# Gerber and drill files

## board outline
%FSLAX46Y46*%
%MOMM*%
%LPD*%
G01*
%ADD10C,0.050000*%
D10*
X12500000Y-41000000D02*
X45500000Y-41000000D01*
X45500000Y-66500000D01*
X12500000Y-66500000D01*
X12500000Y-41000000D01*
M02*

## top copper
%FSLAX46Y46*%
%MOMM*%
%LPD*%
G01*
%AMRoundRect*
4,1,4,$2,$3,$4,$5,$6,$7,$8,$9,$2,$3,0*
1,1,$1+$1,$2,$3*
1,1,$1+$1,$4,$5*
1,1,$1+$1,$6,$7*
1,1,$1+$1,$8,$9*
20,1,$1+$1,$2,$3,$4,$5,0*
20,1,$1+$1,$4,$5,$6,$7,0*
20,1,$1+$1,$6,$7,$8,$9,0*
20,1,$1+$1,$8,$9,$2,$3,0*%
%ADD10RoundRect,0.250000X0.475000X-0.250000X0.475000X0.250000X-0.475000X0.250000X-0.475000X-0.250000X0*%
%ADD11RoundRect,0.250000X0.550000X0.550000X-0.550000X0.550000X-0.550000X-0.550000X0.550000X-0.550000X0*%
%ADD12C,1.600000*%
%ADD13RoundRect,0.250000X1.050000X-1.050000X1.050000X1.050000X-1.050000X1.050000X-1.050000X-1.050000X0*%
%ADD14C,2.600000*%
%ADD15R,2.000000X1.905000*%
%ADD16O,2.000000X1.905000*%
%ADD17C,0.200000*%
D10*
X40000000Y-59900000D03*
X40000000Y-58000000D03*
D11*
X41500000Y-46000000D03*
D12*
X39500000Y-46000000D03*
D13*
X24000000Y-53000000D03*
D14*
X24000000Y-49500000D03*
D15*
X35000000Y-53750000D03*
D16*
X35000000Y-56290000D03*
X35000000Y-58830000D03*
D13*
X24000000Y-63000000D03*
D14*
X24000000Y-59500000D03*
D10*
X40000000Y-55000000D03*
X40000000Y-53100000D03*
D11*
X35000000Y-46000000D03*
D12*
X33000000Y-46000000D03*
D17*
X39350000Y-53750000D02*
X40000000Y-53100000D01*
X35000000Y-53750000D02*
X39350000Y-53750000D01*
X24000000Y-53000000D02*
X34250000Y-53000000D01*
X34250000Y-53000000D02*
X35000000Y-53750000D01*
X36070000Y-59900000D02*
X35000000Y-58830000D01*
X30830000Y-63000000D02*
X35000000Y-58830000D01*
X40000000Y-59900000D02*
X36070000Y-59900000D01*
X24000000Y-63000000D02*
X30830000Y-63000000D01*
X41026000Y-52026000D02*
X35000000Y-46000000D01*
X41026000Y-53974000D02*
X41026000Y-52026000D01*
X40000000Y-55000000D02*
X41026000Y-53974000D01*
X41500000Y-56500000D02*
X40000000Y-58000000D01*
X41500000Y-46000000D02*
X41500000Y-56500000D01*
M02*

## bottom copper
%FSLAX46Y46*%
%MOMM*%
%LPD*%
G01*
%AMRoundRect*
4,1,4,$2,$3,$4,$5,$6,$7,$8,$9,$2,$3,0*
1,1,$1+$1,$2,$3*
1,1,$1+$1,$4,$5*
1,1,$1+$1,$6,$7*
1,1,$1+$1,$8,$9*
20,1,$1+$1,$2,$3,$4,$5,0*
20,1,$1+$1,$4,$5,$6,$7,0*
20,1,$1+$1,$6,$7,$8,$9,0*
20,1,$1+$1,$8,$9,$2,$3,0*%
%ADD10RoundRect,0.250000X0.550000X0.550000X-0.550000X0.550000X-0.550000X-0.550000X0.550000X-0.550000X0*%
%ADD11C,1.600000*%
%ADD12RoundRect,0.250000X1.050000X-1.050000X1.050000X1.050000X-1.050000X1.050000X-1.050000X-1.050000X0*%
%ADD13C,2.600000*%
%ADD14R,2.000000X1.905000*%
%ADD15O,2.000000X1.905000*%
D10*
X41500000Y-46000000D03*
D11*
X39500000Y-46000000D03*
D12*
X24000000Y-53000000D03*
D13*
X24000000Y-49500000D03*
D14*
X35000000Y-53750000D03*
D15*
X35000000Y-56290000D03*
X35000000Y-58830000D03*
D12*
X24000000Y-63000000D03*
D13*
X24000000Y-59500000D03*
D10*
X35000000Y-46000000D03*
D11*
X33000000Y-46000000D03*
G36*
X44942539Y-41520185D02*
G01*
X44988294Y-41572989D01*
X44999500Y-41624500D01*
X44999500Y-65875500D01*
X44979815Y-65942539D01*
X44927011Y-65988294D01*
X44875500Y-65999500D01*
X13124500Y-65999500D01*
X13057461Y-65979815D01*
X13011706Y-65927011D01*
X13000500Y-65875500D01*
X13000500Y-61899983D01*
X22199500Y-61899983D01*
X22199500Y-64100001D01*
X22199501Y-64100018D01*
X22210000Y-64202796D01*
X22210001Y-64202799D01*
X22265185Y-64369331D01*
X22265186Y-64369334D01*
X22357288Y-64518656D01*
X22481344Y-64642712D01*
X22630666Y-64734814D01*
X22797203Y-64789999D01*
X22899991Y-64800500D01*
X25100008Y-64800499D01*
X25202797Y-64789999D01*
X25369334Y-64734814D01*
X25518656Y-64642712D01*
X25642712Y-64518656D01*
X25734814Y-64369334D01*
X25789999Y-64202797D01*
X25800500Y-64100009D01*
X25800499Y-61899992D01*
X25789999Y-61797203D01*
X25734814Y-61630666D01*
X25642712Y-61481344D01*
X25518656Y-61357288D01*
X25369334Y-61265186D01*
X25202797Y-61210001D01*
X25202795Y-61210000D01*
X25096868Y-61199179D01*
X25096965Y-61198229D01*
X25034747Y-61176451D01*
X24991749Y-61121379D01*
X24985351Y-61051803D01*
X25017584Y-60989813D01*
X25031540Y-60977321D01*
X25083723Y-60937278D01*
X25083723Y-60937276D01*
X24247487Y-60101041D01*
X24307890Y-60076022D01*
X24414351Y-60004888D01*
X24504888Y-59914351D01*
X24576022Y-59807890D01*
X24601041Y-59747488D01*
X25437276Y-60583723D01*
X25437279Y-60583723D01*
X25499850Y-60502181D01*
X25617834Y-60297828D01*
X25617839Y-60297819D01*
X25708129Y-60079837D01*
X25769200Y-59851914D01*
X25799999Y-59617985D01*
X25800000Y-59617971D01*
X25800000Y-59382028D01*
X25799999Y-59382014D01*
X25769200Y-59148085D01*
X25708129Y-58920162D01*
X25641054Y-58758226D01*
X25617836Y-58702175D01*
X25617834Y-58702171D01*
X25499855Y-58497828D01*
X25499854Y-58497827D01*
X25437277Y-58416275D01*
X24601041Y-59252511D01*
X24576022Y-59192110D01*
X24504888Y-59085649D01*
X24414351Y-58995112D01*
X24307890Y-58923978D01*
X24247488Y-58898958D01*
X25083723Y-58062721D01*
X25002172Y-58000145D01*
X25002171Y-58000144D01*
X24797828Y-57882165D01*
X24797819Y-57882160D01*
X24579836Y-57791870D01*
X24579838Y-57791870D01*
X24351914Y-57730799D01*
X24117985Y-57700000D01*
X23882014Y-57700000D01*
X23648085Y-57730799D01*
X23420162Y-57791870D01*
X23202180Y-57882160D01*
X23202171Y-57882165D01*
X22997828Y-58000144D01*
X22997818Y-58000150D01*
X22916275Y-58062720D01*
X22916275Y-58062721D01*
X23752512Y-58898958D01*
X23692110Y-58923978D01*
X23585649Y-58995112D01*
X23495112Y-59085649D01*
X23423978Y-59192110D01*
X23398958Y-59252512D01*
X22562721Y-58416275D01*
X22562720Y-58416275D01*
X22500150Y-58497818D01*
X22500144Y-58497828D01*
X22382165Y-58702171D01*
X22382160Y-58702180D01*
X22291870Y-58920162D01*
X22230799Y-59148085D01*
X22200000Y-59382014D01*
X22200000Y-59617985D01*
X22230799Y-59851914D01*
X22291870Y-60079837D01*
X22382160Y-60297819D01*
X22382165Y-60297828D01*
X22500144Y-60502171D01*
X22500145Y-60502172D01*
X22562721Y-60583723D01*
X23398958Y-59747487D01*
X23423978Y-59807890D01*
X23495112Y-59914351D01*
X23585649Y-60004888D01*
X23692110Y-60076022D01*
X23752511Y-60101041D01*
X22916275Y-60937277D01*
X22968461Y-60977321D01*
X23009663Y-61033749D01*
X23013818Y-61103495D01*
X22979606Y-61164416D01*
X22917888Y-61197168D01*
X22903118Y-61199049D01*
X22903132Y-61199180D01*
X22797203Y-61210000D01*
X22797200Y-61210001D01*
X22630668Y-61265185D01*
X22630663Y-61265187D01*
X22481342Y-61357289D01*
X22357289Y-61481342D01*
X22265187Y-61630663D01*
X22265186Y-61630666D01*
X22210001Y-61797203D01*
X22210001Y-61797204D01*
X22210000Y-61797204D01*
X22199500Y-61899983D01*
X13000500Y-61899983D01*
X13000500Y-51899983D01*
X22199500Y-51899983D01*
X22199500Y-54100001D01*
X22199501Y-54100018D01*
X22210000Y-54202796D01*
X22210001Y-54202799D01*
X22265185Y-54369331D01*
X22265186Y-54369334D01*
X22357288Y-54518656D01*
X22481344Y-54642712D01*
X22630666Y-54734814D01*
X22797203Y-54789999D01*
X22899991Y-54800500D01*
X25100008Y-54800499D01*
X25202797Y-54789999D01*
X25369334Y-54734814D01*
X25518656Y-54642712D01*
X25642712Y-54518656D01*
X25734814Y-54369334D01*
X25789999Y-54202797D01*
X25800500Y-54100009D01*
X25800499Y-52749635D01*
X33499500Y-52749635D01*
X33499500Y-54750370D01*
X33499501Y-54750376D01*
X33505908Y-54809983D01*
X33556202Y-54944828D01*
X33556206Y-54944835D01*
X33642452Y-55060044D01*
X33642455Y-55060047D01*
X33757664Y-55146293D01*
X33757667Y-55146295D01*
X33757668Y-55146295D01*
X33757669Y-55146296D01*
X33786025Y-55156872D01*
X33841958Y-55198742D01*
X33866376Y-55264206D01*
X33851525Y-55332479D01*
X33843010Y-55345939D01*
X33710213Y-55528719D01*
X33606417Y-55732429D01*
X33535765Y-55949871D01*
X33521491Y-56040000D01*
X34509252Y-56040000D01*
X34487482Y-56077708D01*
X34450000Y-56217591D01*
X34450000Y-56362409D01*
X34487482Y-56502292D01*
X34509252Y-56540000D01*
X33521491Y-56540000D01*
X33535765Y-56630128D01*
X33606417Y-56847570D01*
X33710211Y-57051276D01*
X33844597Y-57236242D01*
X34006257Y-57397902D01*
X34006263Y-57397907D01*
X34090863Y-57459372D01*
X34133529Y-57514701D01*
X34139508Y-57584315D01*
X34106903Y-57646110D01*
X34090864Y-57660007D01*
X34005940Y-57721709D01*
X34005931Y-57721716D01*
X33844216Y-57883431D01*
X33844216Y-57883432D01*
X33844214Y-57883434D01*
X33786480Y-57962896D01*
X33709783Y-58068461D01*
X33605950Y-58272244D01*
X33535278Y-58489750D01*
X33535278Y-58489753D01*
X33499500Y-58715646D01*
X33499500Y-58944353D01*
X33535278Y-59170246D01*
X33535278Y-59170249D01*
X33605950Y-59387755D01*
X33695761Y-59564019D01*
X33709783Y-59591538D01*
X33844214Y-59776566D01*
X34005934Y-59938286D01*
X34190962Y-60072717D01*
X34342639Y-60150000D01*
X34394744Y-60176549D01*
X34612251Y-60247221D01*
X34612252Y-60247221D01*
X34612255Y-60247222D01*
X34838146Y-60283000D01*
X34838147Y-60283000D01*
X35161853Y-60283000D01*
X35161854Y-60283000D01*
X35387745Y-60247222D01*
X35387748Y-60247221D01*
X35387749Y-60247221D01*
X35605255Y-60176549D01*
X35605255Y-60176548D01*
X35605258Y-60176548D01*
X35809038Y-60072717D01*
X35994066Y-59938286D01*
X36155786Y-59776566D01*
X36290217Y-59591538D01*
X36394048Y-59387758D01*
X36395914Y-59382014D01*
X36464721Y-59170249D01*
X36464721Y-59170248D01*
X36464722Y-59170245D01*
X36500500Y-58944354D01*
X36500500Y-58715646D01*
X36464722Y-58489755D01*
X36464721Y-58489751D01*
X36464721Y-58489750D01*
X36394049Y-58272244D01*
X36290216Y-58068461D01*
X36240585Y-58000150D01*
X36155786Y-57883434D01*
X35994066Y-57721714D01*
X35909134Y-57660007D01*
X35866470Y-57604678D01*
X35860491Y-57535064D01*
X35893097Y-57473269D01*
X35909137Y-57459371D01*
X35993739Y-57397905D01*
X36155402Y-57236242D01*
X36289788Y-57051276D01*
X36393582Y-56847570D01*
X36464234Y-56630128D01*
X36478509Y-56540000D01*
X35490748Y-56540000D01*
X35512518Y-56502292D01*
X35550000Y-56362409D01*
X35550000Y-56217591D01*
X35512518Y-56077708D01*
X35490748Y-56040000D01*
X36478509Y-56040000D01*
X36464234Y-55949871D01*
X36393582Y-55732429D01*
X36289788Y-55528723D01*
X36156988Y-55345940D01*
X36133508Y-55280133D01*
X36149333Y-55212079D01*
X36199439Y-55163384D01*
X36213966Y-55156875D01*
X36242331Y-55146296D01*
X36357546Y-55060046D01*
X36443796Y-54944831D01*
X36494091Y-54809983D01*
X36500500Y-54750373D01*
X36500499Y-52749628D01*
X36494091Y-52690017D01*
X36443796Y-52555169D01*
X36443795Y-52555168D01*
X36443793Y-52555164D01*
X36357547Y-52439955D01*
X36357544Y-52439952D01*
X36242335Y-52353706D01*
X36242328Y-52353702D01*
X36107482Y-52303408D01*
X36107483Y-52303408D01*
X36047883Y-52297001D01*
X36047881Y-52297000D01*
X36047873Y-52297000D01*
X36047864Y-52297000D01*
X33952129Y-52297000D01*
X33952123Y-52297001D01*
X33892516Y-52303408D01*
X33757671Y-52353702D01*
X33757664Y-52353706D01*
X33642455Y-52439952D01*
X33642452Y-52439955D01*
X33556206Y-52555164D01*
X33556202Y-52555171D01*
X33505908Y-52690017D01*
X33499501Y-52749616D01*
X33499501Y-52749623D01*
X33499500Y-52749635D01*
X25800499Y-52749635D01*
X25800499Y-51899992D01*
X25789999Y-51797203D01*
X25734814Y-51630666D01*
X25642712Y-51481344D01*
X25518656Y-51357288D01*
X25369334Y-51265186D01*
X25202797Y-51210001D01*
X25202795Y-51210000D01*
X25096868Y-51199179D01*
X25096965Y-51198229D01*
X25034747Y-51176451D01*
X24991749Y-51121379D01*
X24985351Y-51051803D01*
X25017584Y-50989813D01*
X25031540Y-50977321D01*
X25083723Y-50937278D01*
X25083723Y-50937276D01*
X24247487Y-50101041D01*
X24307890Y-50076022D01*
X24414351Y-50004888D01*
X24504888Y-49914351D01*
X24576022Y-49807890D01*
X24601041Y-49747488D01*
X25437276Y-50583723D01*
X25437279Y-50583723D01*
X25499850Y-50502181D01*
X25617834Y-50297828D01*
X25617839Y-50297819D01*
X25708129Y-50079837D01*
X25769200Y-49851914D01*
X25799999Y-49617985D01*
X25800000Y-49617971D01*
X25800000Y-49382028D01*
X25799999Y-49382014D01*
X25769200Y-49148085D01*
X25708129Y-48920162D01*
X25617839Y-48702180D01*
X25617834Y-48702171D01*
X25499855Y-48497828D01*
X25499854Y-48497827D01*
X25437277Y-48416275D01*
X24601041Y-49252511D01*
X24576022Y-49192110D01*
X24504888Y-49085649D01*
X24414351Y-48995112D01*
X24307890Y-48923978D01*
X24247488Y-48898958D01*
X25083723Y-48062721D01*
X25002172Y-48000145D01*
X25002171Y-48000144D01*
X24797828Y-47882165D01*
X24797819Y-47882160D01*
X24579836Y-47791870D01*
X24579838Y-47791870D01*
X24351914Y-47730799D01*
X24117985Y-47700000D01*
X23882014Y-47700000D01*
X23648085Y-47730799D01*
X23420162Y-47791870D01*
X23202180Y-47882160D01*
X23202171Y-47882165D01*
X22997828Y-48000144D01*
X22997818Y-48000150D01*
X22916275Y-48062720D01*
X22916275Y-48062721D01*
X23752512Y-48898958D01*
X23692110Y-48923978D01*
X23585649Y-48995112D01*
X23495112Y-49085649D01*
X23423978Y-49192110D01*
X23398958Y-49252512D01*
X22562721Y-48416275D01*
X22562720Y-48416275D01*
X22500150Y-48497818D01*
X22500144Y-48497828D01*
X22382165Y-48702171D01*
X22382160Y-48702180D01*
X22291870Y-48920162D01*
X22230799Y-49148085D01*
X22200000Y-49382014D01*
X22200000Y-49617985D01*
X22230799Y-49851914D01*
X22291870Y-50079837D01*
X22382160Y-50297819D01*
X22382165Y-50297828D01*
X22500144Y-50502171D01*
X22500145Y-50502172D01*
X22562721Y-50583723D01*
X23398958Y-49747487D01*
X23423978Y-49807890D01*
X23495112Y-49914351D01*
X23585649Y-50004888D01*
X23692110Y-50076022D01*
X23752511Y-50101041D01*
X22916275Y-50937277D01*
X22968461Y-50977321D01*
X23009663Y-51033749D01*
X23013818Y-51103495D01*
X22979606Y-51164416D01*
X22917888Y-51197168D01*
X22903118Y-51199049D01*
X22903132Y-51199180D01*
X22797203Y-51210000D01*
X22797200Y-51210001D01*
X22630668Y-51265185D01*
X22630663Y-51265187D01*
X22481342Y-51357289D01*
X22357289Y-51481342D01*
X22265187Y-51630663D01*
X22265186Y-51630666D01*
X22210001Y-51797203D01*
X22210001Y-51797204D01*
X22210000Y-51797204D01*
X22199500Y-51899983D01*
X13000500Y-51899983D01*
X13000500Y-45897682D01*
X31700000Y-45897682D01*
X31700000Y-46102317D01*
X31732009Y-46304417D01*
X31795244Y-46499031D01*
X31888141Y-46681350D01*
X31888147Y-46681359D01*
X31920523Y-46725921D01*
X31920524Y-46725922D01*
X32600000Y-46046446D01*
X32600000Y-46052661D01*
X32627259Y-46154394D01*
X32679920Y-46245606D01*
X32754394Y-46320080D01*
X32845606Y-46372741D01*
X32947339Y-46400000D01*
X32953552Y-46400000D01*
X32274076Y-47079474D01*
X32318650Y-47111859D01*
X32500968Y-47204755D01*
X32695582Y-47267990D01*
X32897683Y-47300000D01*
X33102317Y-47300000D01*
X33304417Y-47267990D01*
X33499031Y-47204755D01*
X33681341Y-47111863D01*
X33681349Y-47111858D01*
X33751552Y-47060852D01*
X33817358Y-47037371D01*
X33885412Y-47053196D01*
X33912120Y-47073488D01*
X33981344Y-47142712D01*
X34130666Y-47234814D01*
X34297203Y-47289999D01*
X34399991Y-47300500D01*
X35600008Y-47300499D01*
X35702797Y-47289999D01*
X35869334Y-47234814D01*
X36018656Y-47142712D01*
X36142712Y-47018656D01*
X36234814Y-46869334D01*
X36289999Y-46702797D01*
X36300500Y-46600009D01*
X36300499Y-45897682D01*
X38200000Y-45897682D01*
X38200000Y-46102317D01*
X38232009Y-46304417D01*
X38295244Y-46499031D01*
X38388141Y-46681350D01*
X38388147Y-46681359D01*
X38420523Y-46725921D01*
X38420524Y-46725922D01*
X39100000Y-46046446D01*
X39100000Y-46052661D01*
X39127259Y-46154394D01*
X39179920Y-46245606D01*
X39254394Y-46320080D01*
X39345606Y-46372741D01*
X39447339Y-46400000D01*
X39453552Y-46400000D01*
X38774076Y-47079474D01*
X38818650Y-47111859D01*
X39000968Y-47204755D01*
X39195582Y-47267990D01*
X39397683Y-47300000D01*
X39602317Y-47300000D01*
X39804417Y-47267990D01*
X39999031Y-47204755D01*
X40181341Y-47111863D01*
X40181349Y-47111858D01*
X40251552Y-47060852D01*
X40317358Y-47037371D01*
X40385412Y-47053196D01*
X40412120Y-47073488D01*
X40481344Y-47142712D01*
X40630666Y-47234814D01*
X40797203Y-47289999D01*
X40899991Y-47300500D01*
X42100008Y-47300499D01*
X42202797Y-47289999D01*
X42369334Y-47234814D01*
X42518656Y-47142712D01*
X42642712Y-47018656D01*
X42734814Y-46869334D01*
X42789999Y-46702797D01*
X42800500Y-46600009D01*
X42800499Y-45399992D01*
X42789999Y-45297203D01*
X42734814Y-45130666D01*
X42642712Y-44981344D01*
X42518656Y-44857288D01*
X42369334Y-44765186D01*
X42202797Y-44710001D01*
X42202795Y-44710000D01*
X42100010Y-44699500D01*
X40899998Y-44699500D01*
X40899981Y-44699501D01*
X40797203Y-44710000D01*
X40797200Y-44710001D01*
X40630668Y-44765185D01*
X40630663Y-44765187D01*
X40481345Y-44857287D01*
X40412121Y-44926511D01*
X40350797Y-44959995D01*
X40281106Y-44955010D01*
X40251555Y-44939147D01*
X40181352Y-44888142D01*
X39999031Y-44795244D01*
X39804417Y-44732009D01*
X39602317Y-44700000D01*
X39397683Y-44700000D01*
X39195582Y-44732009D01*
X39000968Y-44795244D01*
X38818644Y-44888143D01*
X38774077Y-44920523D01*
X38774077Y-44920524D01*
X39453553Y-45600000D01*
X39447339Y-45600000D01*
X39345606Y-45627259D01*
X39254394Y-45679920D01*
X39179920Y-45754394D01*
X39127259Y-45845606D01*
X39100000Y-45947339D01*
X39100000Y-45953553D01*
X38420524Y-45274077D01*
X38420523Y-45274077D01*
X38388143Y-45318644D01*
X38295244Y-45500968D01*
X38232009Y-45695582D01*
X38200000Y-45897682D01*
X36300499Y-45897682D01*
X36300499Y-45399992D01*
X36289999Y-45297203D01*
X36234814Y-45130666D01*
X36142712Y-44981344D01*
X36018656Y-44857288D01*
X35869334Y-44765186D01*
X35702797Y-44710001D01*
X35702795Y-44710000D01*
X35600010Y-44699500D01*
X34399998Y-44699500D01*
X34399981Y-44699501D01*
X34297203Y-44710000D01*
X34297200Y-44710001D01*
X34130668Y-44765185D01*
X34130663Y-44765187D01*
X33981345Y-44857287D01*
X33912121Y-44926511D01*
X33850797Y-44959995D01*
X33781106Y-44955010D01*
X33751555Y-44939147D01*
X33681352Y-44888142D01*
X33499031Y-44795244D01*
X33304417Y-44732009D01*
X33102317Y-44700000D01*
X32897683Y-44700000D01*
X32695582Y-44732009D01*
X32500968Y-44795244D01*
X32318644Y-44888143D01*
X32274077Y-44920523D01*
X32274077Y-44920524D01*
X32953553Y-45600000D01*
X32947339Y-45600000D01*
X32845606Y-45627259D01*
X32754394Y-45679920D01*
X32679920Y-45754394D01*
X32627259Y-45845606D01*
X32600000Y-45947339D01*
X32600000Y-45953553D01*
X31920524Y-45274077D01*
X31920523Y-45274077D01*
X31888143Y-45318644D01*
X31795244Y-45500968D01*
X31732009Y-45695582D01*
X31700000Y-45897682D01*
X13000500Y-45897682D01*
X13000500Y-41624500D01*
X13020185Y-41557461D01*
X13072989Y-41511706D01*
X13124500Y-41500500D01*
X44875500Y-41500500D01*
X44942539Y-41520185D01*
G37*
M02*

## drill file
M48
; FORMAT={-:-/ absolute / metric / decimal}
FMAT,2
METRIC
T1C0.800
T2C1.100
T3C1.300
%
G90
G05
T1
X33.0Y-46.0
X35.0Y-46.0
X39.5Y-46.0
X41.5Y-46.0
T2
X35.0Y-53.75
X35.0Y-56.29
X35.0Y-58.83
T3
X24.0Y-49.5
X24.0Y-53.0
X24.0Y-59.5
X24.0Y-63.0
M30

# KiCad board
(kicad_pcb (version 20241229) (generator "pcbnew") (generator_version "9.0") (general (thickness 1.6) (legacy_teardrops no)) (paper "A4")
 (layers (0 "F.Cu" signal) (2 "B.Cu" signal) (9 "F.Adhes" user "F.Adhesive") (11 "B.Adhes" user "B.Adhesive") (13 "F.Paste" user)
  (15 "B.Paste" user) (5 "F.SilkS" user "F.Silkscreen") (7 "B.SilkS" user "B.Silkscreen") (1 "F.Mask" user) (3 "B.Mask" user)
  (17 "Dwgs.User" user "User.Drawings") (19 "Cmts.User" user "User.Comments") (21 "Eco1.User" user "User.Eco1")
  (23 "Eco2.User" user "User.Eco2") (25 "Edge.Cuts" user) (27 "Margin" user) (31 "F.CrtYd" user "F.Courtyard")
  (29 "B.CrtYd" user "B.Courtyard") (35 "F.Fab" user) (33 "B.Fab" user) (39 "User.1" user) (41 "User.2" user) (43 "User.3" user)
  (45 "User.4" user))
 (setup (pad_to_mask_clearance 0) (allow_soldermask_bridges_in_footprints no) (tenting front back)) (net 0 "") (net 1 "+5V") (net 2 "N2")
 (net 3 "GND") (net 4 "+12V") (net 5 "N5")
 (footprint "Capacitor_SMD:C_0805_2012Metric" (layer "F.Cu") (at 40 58.95 90)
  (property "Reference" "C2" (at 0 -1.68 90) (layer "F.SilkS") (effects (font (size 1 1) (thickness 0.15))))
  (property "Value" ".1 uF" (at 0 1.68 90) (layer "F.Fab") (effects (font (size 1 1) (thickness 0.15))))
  (pad "1" smd roundrect (at -0.95 0 90) (size 1 1.45) (layers "F.Cu" "F.Mask" "F.Paste") (roundrect_rratio 0.25) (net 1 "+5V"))
  (pad "2" smd roundrect (at 0.95 0 90) (size 1 1.45) (layers "F.Cu" "F.Mask" "F.Paste") (roundrect_rratio 0.25) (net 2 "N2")))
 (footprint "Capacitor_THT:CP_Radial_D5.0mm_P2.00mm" (layer "F.Cu") (at 41.5 46 180)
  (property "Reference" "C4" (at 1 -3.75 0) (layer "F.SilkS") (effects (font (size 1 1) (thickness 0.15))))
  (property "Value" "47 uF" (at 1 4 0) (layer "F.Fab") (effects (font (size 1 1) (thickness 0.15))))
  (pad "1" thru_hole roundrect (at 0 0 180) (size 1.6 1.6) (drill 0.8) (layers "*.Cu" "*.Mask") (remove_unused_layers no)
   (roundrect_rratio 0.15625) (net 2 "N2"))
  (pad "2" thru_hole circle (at 2 0 180) (size 1.6 1.6) (drill 0.8) (layers "*.Cu" "*.Mask") (remove_unused_layers no) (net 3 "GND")))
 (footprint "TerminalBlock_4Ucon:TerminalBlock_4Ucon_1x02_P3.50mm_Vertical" (layer "F.Cu") (at 24 53 90)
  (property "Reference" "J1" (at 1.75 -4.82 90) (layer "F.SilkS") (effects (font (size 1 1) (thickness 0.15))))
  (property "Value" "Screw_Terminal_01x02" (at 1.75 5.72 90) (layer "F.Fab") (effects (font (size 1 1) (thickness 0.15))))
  (pad "1" thru_hole roundrect (at 0 0 90) (size 2.6 2.6) (drill 1.3) (layers "*.Cu" "*.Mask") (remove_unused_layers no)
   (roundrect_rratio 0.096154) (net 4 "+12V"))
  (pad "2" thru_hole circle (at 3.5 0 90) (size 2.6 2.6) (drill 1.3) (layers "*.Cu" "*.Mask") (remove_unused_layers no) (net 3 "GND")))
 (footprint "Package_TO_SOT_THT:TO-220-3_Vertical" (layer "F.Cu") (at 35 53.75 -90)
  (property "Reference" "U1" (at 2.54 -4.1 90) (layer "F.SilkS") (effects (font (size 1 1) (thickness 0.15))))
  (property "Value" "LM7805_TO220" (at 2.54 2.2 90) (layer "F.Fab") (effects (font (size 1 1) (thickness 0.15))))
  (pad "1" thru_hole rect (at 0 0 270) (size 1.905 2) (drill 1.1) (layers "*.Cu" "*.Mask") (remove_unused_layers no) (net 4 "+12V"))
  (pad "2" thru_hole oval (at 2.54 0 270) (size 1.905 2) (drill 1.1) (layers "*.Cu" "*.Mask") (remove_unused_layers no) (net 3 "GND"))
  (pad "3" thru_hole oval (at 5.08 0 270) (size 1.905 2) (drill 1.1) (layers "*.Cu" "*.Mask") (remove_unused_layers no) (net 1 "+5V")))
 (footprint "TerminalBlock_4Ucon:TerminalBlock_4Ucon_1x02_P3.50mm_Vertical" (layer "F.Cu") (at 24 63 90)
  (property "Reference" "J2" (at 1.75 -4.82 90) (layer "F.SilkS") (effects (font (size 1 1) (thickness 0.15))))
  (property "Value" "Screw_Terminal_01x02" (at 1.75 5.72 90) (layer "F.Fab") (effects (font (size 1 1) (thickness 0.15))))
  (pad "1" thru_hole roundrect (at 0 0 90) (size 2.6 2.6) (drill 1.3) (layers "*.Cu" "*.Mask") (remove_unused_layers no)
   (roundrect_rratio 0.096154) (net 1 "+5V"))
  (pad "2" thru_hole circle (at 3.5 0 90) (size 2.6 2.6) (drill 1.3) (layers "*.Cu" "*.Mask") (remove_unused_layers no) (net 3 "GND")))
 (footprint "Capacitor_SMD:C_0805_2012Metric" (layer "F.Cu") (at 40 54.05 90)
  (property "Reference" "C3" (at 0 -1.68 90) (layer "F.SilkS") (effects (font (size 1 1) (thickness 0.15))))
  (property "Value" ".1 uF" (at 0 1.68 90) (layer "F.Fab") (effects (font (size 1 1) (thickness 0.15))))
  (pad "1" smd roundrect (at -0.95 0 90) (size 1 1.45) (layers "F.Cu" "F.Mask" "F.Paste") (roundrect_rratio 0.25) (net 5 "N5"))
  (pad "2" smd roundrect (at 0.95 0 90) (size 1 1.45) (layers "F.Cu" "F.Mask" "F.Paste") (roundrect_rratio 0.25) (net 4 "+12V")))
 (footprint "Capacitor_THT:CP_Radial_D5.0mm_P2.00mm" (layer "F.Cu") (at 35 46 180)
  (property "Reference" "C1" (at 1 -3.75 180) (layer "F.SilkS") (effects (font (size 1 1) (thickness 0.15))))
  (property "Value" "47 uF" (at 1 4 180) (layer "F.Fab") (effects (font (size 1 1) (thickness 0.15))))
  (pad "1" thru_hole roundrect (at 0 0 180) (size 1.6 1.6) (drill 0.8) (layers "*.Cu" "*.Mask") (remove_unused_layers no)
   (roundrect_rratio 0.15625) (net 5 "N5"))
  (pad "2" thru_hole circle (at 2 0 180) (size 1.6 1.6) (drill 0.8) (layers "*.Cu" "*.Mask") (remove_unused_layers no) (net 3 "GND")))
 (gr_rect (start 12.5 41) (end 45.5 66.5) (stroke (width 0.05) (type default)) (fill no) (layer "Edge.Cuts"))
 (segment (start 39.35 53.75) (end 40 53.1) (width 0.2) (layer "F.Cu") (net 4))
 (segment (start 35 53.75) (end 39.35 53.75) (width 0.2) (layer "F.Cu") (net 4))
 (segment (start 24 53) (end 34.25 53) (width 0.2) (layer "F.Cu") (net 4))
 (segment (start 34.25 53) (end 35 53.75) (width 0.2) (layer "F.Cu") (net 4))
 (segment (start 36.07 59.9) (end 35 58.83) (width 0.2) (layer "F.Cu") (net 1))
 (segment (start 30.83 63) (end 35 58.83) (width 0.2) (layer "F.Cu") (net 1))
 (segment (start 40 59.9) (end 36.07 59.9) (width 0.2) (layer "F.Cu") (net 1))
 (segment (start 24 63) (end 30.83 63) (width 0.2) (layer "F.Cu") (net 1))
 (segment (start 41.026 52.026) (end 35 46) (width 0.2) (layer "F.Cu") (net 5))
 (segment (start 41.026 53.974) (end 41.026 52.026) (width 0.2) (layer "F.Cu") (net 5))
 (segment (start 40 55) (end 41.026 53.974) (width 0.2) (layer "F.Cu") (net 5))
 (segment (start 41.5 56.5) (end 40 58) (width 0.2) (layer "F.Cu") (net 2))
 (segment (start 41.5 46) (end 41.5 56.5) (width 0.2) (layer "F.Cu") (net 2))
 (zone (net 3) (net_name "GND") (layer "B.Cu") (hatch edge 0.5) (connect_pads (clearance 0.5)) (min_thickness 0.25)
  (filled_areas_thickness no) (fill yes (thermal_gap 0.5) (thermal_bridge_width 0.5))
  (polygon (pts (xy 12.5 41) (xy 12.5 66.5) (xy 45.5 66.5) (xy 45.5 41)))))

